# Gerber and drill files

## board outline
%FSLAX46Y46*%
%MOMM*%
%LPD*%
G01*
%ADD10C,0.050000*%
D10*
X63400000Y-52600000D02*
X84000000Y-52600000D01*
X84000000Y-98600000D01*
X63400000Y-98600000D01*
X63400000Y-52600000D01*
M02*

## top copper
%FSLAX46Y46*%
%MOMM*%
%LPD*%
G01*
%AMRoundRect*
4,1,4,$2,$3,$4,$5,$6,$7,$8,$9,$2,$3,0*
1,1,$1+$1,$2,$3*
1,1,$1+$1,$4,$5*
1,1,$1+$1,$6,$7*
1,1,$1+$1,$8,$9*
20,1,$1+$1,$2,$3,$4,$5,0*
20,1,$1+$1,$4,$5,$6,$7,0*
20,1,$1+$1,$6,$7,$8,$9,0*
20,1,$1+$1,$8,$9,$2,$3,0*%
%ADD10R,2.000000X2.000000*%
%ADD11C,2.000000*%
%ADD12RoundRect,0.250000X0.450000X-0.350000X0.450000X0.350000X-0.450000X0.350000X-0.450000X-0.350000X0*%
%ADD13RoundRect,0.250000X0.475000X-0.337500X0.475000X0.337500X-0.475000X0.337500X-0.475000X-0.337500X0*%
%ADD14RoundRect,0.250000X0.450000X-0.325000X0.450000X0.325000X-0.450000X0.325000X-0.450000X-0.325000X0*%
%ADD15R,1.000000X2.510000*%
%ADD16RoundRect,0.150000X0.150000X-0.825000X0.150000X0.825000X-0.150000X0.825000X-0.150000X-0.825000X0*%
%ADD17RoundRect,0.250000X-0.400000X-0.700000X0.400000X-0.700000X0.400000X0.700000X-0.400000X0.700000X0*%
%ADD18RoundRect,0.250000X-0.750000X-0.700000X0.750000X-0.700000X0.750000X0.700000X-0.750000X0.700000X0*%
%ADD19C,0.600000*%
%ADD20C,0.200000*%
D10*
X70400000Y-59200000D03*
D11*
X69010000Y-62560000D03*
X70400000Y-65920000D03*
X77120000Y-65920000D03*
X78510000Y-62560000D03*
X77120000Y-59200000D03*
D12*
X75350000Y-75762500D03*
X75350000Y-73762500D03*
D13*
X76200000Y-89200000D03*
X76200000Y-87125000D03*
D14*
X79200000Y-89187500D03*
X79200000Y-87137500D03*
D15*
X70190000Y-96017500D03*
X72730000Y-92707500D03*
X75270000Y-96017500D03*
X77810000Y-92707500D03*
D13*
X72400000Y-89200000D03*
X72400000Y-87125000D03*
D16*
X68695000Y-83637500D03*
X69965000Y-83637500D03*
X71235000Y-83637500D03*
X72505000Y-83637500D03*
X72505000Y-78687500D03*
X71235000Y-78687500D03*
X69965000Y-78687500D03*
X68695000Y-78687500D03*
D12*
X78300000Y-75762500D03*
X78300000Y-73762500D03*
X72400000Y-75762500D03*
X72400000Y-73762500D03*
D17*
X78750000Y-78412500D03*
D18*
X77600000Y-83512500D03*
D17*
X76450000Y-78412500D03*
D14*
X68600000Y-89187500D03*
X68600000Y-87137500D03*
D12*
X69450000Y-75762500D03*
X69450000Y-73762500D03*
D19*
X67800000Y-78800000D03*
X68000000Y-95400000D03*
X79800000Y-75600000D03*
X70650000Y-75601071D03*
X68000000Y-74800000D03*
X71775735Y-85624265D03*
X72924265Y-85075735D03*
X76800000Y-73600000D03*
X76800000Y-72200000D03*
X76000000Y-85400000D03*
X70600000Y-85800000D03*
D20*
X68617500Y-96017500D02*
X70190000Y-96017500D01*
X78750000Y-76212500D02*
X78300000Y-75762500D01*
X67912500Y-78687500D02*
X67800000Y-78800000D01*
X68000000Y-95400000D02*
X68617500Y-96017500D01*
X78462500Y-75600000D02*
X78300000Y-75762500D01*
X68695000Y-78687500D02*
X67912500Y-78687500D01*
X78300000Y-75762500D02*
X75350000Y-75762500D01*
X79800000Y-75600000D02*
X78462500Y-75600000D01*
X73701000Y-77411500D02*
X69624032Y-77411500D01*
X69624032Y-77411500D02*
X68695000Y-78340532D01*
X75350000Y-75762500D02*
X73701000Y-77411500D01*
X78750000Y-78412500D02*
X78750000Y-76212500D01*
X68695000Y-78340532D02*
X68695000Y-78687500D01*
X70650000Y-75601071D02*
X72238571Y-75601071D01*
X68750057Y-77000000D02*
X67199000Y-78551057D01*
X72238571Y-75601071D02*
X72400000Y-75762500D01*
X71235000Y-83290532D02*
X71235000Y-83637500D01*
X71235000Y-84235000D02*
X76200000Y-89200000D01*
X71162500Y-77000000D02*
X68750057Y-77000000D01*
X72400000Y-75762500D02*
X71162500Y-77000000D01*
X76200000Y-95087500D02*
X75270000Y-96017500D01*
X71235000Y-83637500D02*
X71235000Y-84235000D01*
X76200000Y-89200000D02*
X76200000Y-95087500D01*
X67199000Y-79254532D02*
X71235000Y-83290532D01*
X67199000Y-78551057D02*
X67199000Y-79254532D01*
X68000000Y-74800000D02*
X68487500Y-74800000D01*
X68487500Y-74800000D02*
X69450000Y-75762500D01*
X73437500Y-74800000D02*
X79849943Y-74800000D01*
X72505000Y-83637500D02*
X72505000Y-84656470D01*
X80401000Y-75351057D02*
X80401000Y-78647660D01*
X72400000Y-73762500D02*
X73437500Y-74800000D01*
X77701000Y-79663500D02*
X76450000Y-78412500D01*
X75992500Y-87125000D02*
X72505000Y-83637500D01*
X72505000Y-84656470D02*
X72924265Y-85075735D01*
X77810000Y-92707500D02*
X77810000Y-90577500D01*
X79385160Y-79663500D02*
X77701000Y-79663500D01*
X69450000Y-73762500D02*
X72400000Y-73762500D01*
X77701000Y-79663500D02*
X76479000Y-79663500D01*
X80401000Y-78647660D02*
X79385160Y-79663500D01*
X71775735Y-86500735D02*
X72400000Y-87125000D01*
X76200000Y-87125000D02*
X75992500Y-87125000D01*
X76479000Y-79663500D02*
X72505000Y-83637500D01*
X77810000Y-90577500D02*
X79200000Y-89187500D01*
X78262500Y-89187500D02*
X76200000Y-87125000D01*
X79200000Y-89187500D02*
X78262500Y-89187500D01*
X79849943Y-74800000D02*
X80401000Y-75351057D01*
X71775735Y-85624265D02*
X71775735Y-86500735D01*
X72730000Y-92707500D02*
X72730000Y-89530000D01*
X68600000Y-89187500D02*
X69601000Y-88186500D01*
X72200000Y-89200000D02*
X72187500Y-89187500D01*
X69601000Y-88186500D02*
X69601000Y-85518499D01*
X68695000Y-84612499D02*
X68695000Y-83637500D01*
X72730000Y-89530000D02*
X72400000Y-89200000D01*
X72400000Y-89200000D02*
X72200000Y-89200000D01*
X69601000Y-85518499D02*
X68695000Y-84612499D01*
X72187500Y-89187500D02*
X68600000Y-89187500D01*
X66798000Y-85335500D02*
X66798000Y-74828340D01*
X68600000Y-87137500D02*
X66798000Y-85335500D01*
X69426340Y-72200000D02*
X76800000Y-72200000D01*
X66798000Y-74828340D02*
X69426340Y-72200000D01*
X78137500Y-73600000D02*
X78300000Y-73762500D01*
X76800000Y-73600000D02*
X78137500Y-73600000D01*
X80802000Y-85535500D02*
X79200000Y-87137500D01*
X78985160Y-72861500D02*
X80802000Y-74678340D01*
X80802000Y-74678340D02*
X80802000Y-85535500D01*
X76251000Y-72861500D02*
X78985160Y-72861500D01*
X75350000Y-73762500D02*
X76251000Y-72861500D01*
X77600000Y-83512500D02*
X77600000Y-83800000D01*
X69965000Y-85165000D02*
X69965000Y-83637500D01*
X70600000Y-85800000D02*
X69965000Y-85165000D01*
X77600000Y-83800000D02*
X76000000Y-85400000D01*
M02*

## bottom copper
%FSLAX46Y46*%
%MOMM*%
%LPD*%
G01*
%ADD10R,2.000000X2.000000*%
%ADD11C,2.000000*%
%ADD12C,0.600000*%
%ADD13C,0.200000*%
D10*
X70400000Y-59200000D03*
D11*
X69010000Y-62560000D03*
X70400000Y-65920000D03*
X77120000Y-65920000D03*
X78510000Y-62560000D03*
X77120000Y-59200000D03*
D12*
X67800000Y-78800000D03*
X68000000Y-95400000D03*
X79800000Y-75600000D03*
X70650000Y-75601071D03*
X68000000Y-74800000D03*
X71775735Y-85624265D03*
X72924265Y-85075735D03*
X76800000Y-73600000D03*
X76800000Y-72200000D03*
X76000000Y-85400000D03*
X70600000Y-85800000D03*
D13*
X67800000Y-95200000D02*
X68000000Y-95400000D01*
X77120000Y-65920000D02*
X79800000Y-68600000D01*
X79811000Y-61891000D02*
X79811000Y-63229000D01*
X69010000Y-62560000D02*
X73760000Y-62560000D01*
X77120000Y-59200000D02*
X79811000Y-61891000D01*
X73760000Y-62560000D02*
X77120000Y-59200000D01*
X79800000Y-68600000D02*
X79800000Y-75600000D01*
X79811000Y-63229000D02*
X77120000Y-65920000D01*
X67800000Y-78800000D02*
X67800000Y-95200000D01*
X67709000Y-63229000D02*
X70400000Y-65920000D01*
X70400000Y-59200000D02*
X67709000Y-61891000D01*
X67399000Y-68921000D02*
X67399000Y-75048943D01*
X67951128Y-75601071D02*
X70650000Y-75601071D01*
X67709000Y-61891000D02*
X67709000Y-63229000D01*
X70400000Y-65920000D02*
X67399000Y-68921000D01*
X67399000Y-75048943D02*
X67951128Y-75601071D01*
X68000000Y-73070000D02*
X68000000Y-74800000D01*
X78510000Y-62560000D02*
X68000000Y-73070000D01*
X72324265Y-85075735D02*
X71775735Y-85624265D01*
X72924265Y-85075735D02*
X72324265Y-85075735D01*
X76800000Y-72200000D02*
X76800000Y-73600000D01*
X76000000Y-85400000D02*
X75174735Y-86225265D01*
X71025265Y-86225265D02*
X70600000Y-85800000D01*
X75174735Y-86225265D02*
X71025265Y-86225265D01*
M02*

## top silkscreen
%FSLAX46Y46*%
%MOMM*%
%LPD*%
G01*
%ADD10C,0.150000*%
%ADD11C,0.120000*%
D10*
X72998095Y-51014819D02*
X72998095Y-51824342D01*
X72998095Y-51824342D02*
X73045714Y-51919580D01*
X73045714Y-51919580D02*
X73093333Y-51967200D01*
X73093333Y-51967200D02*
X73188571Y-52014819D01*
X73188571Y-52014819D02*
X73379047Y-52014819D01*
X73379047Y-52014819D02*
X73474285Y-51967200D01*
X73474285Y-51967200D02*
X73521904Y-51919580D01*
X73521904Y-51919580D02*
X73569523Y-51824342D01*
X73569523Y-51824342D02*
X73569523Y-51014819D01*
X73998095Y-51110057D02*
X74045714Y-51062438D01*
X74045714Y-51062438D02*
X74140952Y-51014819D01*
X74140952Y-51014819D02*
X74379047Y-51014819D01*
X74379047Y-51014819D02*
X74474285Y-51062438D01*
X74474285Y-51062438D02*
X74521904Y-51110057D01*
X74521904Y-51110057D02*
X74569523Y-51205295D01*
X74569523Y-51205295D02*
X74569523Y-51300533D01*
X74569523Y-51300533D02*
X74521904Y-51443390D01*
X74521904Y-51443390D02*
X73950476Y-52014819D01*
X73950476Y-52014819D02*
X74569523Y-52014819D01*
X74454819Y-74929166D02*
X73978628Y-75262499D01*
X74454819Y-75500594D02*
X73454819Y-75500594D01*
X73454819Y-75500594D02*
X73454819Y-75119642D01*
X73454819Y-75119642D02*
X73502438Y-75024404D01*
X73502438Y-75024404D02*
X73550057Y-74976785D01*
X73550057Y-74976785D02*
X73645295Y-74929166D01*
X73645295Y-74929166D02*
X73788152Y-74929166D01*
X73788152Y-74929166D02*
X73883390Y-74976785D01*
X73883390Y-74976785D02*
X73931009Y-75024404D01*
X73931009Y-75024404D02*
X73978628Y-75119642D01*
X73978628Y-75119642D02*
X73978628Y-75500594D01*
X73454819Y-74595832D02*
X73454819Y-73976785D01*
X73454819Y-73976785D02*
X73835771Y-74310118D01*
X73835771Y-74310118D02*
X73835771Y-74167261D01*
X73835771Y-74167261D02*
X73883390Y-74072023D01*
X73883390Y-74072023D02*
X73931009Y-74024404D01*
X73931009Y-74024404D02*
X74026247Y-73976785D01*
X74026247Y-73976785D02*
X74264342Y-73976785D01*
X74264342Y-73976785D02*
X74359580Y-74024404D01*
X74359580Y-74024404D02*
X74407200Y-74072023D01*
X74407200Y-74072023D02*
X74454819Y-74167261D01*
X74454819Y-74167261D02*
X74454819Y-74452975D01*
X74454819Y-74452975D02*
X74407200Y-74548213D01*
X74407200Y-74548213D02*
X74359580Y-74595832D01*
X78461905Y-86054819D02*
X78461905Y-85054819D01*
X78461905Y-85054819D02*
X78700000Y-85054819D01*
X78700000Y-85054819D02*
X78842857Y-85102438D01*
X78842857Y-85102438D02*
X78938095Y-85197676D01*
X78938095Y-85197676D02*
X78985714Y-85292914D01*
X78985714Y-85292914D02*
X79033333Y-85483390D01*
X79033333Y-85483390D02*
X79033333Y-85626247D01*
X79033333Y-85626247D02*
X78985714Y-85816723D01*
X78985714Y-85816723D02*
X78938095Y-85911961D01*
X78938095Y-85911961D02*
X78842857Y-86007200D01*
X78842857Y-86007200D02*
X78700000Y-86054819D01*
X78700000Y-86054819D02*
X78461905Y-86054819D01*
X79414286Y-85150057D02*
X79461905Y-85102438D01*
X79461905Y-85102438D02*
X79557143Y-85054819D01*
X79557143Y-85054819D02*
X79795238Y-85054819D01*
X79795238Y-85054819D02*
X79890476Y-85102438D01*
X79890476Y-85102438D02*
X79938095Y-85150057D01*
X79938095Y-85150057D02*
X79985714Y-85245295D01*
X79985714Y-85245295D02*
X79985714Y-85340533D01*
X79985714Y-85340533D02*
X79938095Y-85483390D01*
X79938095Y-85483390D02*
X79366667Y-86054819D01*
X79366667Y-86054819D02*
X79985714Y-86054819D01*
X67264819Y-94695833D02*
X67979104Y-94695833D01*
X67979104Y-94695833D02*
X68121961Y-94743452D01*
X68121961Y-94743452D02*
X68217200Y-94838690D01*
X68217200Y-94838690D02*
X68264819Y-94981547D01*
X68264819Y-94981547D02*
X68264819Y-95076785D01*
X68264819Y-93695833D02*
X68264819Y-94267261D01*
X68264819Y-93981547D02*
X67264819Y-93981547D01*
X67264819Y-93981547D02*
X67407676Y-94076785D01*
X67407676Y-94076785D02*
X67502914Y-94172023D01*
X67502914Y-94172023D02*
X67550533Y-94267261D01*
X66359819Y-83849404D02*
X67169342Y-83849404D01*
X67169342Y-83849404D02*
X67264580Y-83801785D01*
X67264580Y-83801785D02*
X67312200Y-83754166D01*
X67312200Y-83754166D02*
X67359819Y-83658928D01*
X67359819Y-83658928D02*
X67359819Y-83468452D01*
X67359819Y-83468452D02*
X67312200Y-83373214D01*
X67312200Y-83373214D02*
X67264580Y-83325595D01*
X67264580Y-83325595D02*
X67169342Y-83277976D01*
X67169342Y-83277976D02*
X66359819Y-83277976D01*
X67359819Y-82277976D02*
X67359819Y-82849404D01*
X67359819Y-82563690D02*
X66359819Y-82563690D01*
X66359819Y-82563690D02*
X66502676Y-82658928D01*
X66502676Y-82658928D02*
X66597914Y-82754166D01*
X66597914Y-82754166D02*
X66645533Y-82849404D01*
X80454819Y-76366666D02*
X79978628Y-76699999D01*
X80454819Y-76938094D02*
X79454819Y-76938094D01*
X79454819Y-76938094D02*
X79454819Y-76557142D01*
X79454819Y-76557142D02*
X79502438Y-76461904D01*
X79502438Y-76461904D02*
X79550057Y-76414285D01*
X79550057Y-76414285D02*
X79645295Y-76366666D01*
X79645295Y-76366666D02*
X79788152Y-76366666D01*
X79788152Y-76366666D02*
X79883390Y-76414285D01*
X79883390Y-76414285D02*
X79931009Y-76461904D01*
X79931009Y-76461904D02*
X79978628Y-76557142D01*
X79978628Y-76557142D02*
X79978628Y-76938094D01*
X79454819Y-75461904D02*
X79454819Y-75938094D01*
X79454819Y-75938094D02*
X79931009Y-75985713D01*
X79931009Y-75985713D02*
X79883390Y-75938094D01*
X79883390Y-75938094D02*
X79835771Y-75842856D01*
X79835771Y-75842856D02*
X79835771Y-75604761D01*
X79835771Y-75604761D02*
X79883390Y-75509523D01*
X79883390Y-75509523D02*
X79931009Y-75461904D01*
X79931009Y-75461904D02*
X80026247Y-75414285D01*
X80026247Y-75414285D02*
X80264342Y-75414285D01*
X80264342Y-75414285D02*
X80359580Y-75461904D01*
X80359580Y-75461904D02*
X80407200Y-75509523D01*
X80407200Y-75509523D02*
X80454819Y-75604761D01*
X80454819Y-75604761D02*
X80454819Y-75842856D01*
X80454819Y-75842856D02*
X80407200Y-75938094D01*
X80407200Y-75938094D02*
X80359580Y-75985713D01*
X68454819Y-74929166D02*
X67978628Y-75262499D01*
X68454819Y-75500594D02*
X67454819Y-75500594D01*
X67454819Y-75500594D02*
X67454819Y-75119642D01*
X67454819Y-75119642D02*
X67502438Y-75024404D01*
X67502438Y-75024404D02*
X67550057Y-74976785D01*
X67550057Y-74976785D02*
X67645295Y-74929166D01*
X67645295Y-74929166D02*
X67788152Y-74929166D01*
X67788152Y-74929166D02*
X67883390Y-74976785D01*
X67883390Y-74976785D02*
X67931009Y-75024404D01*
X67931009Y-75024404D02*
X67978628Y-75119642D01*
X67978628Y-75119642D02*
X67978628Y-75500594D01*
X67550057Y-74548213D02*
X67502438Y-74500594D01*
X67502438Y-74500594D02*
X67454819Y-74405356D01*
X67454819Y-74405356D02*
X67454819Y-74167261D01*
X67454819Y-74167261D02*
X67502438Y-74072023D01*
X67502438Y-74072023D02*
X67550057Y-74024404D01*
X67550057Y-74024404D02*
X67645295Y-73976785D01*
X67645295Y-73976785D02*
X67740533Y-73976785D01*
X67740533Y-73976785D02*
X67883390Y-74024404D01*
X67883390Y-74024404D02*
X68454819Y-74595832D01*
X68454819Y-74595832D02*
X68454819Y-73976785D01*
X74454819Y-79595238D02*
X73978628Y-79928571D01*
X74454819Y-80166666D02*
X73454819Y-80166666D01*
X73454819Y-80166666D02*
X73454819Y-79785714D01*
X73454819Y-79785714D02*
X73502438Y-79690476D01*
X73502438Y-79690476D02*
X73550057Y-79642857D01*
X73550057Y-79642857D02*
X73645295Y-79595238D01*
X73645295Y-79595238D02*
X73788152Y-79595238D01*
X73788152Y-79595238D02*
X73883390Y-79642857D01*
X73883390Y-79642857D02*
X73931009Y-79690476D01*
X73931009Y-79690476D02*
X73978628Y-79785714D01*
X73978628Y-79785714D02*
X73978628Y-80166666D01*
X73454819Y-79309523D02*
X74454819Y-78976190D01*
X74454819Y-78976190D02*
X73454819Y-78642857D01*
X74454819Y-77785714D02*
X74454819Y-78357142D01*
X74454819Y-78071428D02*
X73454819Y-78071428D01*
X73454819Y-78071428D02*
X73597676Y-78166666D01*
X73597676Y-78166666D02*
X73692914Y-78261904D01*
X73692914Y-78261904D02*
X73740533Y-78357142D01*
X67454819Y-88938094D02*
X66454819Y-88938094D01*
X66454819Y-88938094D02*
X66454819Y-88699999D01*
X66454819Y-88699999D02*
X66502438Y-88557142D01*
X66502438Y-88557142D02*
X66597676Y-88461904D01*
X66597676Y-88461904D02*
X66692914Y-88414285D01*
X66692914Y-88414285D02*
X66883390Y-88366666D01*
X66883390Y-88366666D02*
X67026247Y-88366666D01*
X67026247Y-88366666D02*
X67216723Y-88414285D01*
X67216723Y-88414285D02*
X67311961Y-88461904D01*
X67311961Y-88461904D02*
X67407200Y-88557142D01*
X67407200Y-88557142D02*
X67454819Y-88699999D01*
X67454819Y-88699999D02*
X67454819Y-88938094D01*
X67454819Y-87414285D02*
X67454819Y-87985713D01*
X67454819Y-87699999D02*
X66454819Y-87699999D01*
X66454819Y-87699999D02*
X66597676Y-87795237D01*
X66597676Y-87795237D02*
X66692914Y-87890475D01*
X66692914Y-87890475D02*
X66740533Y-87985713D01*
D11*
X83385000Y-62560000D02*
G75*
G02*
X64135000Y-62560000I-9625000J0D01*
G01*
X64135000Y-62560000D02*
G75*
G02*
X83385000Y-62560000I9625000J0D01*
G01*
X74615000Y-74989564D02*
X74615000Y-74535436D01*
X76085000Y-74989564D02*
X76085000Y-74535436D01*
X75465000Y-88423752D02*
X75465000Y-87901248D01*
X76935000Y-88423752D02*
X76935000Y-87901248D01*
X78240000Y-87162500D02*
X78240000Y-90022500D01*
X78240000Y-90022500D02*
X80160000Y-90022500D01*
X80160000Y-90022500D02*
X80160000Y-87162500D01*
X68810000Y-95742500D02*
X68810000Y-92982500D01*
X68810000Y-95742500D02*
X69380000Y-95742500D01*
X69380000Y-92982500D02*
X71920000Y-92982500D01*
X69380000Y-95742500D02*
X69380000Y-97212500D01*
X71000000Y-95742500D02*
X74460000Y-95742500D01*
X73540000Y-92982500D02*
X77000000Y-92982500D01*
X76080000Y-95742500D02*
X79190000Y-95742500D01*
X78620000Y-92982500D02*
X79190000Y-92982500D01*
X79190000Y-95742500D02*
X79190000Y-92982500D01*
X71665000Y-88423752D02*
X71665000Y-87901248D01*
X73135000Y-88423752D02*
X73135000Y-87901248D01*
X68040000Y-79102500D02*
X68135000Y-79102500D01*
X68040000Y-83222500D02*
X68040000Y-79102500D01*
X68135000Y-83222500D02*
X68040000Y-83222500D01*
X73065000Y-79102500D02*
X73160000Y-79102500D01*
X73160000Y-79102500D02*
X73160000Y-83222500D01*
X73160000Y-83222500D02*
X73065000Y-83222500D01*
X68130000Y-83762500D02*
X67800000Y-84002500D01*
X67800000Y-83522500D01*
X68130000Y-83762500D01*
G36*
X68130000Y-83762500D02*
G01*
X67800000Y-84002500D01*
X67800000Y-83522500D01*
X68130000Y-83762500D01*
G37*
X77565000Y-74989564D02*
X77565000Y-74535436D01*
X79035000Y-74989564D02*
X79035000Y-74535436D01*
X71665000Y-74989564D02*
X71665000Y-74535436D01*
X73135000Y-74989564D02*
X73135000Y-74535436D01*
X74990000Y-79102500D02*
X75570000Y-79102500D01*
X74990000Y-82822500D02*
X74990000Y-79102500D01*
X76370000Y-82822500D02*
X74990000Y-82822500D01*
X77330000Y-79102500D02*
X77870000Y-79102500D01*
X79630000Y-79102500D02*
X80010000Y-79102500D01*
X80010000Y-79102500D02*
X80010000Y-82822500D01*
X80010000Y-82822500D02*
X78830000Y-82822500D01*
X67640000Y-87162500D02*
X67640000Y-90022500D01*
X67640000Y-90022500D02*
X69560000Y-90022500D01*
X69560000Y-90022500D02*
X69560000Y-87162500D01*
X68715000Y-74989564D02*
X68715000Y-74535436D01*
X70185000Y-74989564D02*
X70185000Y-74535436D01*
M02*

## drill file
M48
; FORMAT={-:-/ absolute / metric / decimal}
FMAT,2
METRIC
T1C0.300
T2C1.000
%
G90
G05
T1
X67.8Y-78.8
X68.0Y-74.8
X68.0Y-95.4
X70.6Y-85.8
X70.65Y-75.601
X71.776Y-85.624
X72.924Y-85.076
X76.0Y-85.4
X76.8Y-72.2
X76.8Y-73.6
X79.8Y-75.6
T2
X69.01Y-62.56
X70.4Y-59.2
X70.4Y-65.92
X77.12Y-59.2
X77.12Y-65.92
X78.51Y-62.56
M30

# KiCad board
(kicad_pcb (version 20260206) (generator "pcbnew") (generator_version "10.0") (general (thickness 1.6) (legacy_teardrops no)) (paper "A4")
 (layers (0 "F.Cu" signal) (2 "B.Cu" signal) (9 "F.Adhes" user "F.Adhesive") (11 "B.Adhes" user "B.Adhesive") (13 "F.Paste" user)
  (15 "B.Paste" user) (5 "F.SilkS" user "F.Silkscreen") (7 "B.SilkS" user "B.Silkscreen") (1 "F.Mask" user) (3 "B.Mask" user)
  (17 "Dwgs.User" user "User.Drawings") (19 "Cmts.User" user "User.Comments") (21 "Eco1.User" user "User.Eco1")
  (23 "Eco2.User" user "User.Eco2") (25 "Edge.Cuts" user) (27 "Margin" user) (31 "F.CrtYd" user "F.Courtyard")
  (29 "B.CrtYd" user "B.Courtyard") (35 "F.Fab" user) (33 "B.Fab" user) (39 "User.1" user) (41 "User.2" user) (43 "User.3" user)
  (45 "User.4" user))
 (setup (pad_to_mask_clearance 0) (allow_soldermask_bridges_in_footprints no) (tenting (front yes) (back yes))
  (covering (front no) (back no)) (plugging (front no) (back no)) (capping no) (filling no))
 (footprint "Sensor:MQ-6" (layer "F.Cu") (at 70.4 59.2)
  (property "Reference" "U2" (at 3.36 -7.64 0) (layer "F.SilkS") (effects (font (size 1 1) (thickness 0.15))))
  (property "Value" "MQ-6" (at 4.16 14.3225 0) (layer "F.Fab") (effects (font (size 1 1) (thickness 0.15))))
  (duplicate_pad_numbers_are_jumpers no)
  (fp_circle (center 3.36 3.36) (end 12.985 3.36) (stroke (width 0.12) (type solid)) (fill no) (layer "F.SilkS"))
  (pad "1" thru_hole rect (at 0 0) (size 2 2) (drill 1) (layers "*.Cu" "*.Mask") (remove_unused_layers no) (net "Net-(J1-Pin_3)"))
  (pad "2" thru_hole circle (at -1.39 3.36) (size 2 2) (drill 1) (layers "*.Cu" "*.Mask") (remove_unused_layers no) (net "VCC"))
  (pad "3" thru_hole circle (at 0 6.72 90) (size 2 2) (drill 1) (layers "*.Cu" "*.Mask") (remove_unused_layers no) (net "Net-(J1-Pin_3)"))
  (pad "4" thru_hole circle (at 6.72 6.72 180) (size 2 2) (drill 1) (layers "*.Cu" "*.Mask") (remove_unused_layers no) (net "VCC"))
  (pad "5" thru_hole circle (at 8.11 3.36) (size 2 2) (drill 1) (layers "*.Cu" "*.Mask") (remove_unused_layers no) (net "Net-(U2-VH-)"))
  (pad "6" thru_hole circle (at 6.72 0 270) (size 2 2) (drill 1) (layers "*.Cu" "*.Mask") (remove_unused_layers no) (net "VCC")))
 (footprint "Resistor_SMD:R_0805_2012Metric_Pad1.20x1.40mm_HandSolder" (layer "F.Cu") (at 75.35 74.7625 90)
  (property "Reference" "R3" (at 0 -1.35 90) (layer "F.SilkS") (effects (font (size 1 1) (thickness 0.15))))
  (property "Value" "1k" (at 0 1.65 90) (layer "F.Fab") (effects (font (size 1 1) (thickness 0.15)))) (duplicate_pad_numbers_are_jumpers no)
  (fp_line (start -0.227064 -0.735) (end 0.227064 -0.735) (stroke (width 0.12) (type solid)) (layer "F.SilkS"))
  (fp_line (start -0.227064 0.735) (end 0.227064 0.735) (stroke (width 0.12) (type solid)) (layer "F.SilkS"))
  (pad "1" smd roundrect (at -1 0 90) (size 1.2 1.4) (layers "F.Cu" "F.Mask" "F.Paste") (roundrect_rratio 0.208333) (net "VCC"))
  (pad "2" smd roundrect (at 1 0 90) (size 1.2 1.4) (layers "F.Cu" "F.Mask" "F.Paste") (roundrect_rratio 0.208333) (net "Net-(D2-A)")))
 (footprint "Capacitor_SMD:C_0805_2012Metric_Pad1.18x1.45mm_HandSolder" (layer "F.Cu") (at 76.2 88.1625 90)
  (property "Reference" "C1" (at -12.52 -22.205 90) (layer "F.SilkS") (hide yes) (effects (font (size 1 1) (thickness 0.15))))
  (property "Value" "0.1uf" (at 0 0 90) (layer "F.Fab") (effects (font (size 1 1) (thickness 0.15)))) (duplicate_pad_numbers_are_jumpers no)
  (fp_line (start -0.261252 -0.735) (end 0.261252 -0.735) (stroke (width 0.12) (type solid)) (layer "F.SilkS"))
  (fp_line (start -0.261252 0.735) (end 0.261252 0.735) (stroke (width 0.12) (type solid)) (layer "F.SilkS"))
  (pad "1" smd roundrect (at -1.0375 0 90) (size 1.175 1.45) (layers "F.Cu" "F.Mask" "F.Paste") (roundrect_rratio 0.212766)
   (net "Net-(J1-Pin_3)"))
  (pad "2" smd roundrect (at 1.0375 0 90) (size 1.175 1.45) (layers "F.Cu" "F.Mask" "F.Paste") (roundrect_rratio 0.212766) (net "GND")))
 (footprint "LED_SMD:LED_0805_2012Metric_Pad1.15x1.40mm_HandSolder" (layer "F.Cu") (at 79.2 88.1625 90)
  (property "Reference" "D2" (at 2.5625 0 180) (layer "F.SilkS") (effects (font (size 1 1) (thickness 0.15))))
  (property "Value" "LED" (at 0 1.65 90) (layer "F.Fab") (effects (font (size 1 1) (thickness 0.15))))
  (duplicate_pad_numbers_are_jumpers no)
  (fp_line (start 1 -0.96) (end -1.86 -0.96) (stroke (width 0.12) (type solid)) (layer "F.SilkS"))
  (fp_line (start -1.86 -0.96) (end -1.86 0.96) (stroke (width 0.12) (type solid)) (layer "F.SilkS"))
  (fp_line (start -1.86 0.96) (end 1 0.96) (stroke (width 0.12) (type solid)) (layer "F.SilkS"))
  (pad "1" smd roundrect (at -1.025 0 90) (size 1.15 1.4) (layers "F.Cu" "F.Mask" "F.Paste") (roundrect_rratio 0.217391) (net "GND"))
  (pad "2" smd roundrect (at 1.025 0 90) (size 1.15 1.4) (layers "F.Cu" "F.Mask" "F.Paste") (roundrect_rratio 0.217391) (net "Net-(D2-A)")))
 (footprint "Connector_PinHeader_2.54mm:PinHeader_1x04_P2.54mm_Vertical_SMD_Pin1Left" (layer "F.Cu") (at 74 94.3625 90)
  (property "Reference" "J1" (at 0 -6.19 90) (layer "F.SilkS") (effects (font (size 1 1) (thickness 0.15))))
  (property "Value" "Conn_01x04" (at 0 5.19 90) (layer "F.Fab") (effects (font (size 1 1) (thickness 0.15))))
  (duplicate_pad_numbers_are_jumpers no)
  (fp_line (start -1.38 -5.19) (end 1.38 -5.19) (stroke (width 0.12) (type solid)) (layer "F.SilkS"))
  (fp_line (start -1.38 -5.19) (end -1.38 -4.62) (stroke (width 0.12) (type solid)) (layer "F.SilkS"))
  (fp_line (start 1.38 -4.62) (end 1.38 -2.08) (stroke (width 0.12) (type solid)) (layer "F.SilkS"))
  (fp_line (start -1.38 -4.62) (end -2.85 -4.62) (stroke (width 0.12) (type solid)) (layer "F.SilkS"))
  (fp_line (start -1.38 -3) (end -1.38 0.46) (stroke (width 0.12) (type solid)) (layer "F.SilkS"))
  (fp_line (start 1.38 -0.46) (end 1.38 3) (stroke (width 0.12) (type solid)) (layer "F.SilkS"))
  (fp_line (start -1.38 2.08) (end -1.38 5.19) (stroke (width 0.12) (type solid)) (layer "F.SilkS"))
  (fp_line (start 1.38 4.62) (end 1.38 5.19) (stroke (width 0.12) (type solid)) (layer "F.SilkS"))
  (fp_line (start -1.38 5.19) (end 1.38 5.19) (stroke (width 0.12) (type solid)) (layer "F.SilkS"))
  (pad "1" smd rect (at -1.655 -3.81 90) (size 2.51 1) (layers "F.Cu" "F.Mask" "F.Paste") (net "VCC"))
  (pad "2" smd rect (at 1.655 -1.27 90) (size 2.51 1) (layers "F.Cu" "F.Mask" "F.Paste") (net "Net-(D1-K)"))
  (pad "3" smd rect (at -1.655 1.27 90) (size 2.51 1) (layers "F.Cu" "F.Mask" "F.Paste") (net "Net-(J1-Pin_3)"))
  (pad "4" smd rect (at 1.655 3.81 90) (size 2.51 1) (layers "F.Cu" "F.Mask" "F.Paste") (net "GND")))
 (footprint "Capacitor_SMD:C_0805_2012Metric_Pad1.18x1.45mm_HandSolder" (layer "F.Cu") (at 72.4 88.1625 90)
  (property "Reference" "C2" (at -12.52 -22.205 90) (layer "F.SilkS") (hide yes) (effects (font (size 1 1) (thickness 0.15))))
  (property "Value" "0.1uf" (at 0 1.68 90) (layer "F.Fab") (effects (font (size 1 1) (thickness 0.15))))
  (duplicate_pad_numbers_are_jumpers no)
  (fp_line (start -0.261252 -0.735) (end 0.261252 -0.735) (stroke (width 0.12) (type solid)) (layer "F.SilkS"))
  (fp_line (start -0.261252 0.735) (end 0.261252 0.735) (stroke (width 0.12) (type solid)) (layer "F.SilkS"))
  (pad "1" smd roundrect (at -1.0375 0 90) (size 1.175 1.45) (layers "F.Cu" "F.Mask" "F.Paste") (roundrect_rratio 0.212766)
   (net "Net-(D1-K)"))
  (pad "2" smd roundrect (at 1.0375 0 90) (size 1.175 1.45) (layers "F.Cu" "F.Mask" "F.Paste") (roundrect_rratio 0.212766) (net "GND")))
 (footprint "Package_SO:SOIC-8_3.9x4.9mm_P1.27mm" (layer "F.Cu") (at 70.6 81.1625 90)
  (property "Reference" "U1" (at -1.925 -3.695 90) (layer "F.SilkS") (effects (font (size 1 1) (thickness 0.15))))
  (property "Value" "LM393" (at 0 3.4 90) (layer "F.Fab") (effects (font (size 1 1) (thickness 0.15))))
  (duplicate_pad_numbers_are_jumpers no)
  (fp_line (start 2.06 -2.56) (end 2.06 -2.465) (stroke (width 0.12) (type solid)) (layer "F.SilkS"))
  (fp_line (start -2.06 -2.56) (end 2.06 -2.56) (stroke (width 0.12) (type solid)) (layer "F.SilkS"))
  (fp_line (start -2.06 -2.465) (end -2.06 -2.56) (stroke (width 0.12) (type solid)) (layer "F.SilkS"))
  (fp_line (start 2.06 2.465) (end 2.06 2.56) (stroke (width 0.12) (type solid)) (layer "F.SilkS"))
  (fp_line (start 2.06 2.56) (end -2.06 2.56) (stroke (width 0.12) (type solid)) (layer "F.SilkS"))
  (fp_line (start -2.06 2.56) (end -2.06 2.465) (stroke (width 0.12) (type solid)) (layer "F.SilkS"))
  (fp_poly (pts (xy -2.6 -2.47) (xy -2.84 -2.8) (xy -2.36 -2.8)) (stroke (width 0.12) (type solid)) (fill yes) (layer "F.SilkS"))
  (pad "1" smd roundrect (at -2.475 -1.905 90) (size 1.95 0.6) (layers "F.Cu" "F.Mask" "F.Paste") (roundrect_rratio 0.25) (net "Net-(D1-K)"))
  (pad "2" smd roundrect (at -2.475 -0.635 90) (size 1.95 0.6) (layers "F.Cu" "F.Mask" "F.Paste") (roundrect_rratio 0.25)
   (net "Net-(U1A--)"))
  (pad "3" smd roundrect (at -2.475 0.635 90) (size 1.95 0.6) (layers "F.Cu" "F.Mask" "F.Paste") (roundrect_rratio 0.25)
   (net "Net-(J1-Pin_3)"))
  (pad "4" smd roundrect (at -2.475 1.905 90) (size 1.95 0.6) (layers "F.Cu" "F.Mask" "F.Paste") (roundrect_rratio 0.25) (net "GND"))
  (pad "5" smd roundrect (at 2.475 1.905 90) (size 1.95 0.6) (layers "F.Cu" "F.Mask" "F.Paste") (roundrect_rratio 0.25))
  (pad "6" smd roundrect (at 2.475 0.635 90) (size 1.95 0.6) (layers "F.Cu" "F.Mask" "F.Paste") (roundrect_rratio 0.25))
  (pad "7" smd roundrect (at 2.475 -0.635 90) (size 1.95 0.6) (layers "F.Cu" "F.Mask" "F.Paste") (roundrect_rratio 0.25))
  (pad "8" smd roundrect (at 2.475 -1.905 90) (size 1.95 0.6) (layers "F.Cu" "F.Mask" "F.Paste") (roundrect_rratio 0.25) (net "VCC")))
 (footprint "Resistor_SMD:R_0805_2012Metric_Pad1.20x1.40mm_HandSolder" (layer "F.Cu") (at 78.3 74.7625 90)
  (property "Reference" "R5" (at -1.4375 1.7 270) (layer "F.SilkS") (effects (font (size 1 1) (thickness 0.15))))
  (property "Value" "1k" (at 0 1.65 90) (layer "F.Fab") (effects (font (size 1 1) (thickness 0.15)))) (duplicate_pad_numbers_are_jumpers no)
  (fp_line (start -0.227064 -0.735) (end 0.227064 -0.735) (stroke (width 0.12) (type solid)) (layer "F.SilkS"))
  (fp_line (start -0.227064 0.735) (end 0.227064 0.735) (stroke (width 0.12) (type solid)) (layer "F.SilkS"))
  (pad "1" smd roundrect (at -1 0 90) (size 1.2 1.4) (layers "F.Cu" "F.Mask" "F.Paste") (roundrect_rratio 0.208333) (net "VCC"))
  (pad "2" smd roundrect (at 1 0 90) (size 1.2 1.4) (layers "F.Cu" "F.Mask" "F.Paste") (roundrect_rratio 0.208333) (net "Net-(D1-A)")))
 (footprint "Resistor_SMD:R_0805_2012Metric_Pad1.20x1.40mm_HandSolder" (layer "F.Cu") (at 72.4 74.7625 90)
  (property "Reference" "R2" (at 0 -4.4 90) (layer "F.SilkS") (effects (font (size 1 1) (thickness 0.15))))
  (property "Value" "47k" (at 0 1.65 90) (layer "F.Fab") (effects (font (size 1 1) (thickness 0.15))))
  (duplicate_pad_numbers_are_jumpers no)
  (fp_line (start -0.227064 -0.735) (end 0.227064 -0.735) (stroke (width 0.12) (type solid)) (layer "F.SilkS"))
  (fp_line (start -0.227064 0.735) (end 0.227064 0.735) (stroke (width 0.12) (type solid)) (layer "F.SilkS"))
  (pad "1" smd roundrect (at -1 0 90) (size 1.2 1.4) (layers "F.Cu" "F.Mask" "F.Paste") (roundrect_rratio 0.208333) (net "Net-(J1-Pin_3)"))
  (pad "2" smd roundrect (at 1 0 90) (size 1.2 1.4) (layers "F.Cu" "F.Mask" "F.Paste") (roundrect_rratio 0.208333) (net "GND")))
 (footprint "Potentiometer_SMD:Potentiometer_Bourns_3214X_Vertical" (layer "F.Cu") (at 77.6 80.9625)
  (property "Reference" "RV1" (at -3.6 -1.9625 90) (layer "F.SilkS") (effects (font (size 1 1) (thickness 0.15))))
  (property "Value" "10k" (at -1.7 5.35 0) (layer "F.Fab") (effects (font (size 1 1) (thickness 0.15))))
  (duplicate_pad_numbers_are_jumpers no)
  (fp_line (start -2.61 -1.86) (end -2.03 -1.86) (stroke (width 0.12) (type solid)) (layer "F.SilkS"))
  (fp_line (start -2.61 1.86) (end -2.61 -1.86) (stroke (width 0.12) (type solid)) (layer "F.SilkS"))
  (fp_line (start -1.23 1.86) (end -2.61 1.86) (stroke (width 0.12) (type solid)) (layer "F.SilkS"))
  (fp_line (start -0.27 -1.86) (end 0.27 -1.86) (stroke (width 0.12) (type solid)) (layer "F.SilkS"))
  (fp_line (start 2.03 -1.86) (end 2.41 -1.86) (stroke (width 0.12) (type solid)) (layer "F.SilkS"))
  (fp_line (start 2.41 -1.86) (end 2.41 1.86) (stroke (width 0.12) (type solid)) (layer "F.SilkS"))
  (fp_line (start 2.41 1.86) (end 1.23 1.86) (stroke (width 0.12) (type solid)) (layer "F.SilkS"))
  (pad "1" smd roundrect (at 1.15 -2.55) (size 1.3 1.9) (layers "F.Cu" "F.Mask" "F.Paste") (roundrect_rratio 0.192308) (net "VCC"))
  (pad "2" smd roundrect (at 0 2.55) (size 2 1.9) (layers "F.Cu" "F.Mask" "F.Paste") (roundrect_rratio 0.131579) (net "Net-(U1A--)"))
  (pad "3" smd roundrect (at -1.15 -2.55) (size 1.3 1.9) (layers "F.Cu" "F.Mask" "F.Paste") (roundrect_rratio 0.192308) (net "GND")))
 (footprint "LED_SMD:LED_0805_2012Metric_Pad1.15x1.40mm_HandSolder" (layer "F.Cu") (at 68.6 88.1625 90)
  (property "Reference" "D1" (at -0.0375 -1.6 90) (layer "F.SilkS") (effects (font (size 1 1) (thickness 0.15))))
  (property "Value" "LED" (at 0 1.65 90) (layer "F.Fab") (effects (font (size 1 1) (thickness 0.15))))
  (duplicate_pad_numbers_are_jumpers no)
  (fp_line (start 1 -0.96) (end -1.86 -0.96) (stroke (width 0.12) (type solid)) (layer "F.SilkS"))
  (fp_line (start -1.86 -0.96) (end -1.86 0.96) (stroke (width 0.12) (type solid)) (layer "F.SilkS"))
  (fp_line (start -1.86 0.96) (end 1 0.96) (stroke (width 0.12) (type solid)) (layer "F.SilkS"))
  (pad "1" smd roundrect (at -1.025 0 90) (size 1.15 1.4) (layers "F.Cu" "F.Mask" "F.Paste") (roundrect_rratio 0.217391) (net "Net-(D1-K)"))
  (pad "2" smd roundrect (at 1.025 0 90) (size 1.15 1.4) (layers "F.Cu" "F.Mask" "F.Paste") (roundrect_rratio 0.217391) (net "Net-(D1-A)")))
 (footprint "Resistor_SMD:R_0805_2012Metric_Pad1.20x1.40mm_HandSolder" (layer "F.Cu") (at 69.45 74.7625 90)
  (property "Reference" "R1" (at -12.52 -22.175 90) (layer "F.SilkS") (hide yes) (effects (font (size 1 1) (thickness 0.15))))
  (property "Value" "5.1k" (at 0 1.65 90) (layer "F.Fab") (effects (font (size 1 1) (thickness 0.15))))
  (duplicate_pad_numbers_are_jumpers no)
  (fp_line (start -0.227064 -0.735) (end 0.227064 -0.735) (stroke (width 0.12) (type solid)) (layer "F.SilkS"))
  (fp_line (start -0.227064 0.735) (end 0.227064 0.735) (stroke (width 0.12) (type solid)) (layer "F.SilkS"))
  (pad "1" smd roundrect (at -1 0 90) (size 1.2 1.4) (layers "F.Cu" "F.Mask" "F.Paste") (roundrect_rratio 0.208333) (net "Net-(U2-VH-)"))
  (pad "2" smd roundrect (at 1 0 90) (size 1.2 1.4) (layers "F.Cu" "F.Mask" "F.Paste") (roundrect_rratio 0.208333) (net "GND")))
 (gr_rect (start 63.4 52.6) (end 84 98.6) (stroke (width 0.05) (type default)) (fill no) (layer "Edge.Cuts"))
 (segment (start 68.6175 96.0175) (end 70.19 96.0175) (width 0.2) (layer "F.Cu") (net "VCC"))
 (segment (start 78.75 76.2125) (end 78.3 75.7625) (width 0.2) (layer "F.Cu") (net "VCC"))
 (segment (start 67.9125 78.6875) (end 67.8 78.8) (width 0.2) (layer "F.Cu") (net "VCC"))
 (segment (start 68 95.4) (end 68.6175 96.0175) (width 0.2) (layer "F.Cu") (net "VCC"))
 (segment (start 78.4625 75.6) (end 78.3 75.7625) (width 0.2) (layer "F.Cu") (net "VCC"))
 (segment (start 68.695 78.6875) (end 67.9125 78.6875) (width 0.2) (layer "F.Cu") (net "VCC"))
 (segment (start 78.3 75.7625) (end 75.35 75.7625) (width 0.2) (layer "F.Cu") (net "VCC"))
 (segment (start 79.8 75.6) (end 78.4625 75.6) (width 0.2) (layer "F.Cu") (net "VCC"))
 (segment (start 73.701 77.4115) (end 69.624032 77.4115) (width 0.2) (layer "F.Cu") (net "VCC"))
 (segment (start 69.624032 77.4115) (end 68.695 78.340532) (width 0.2) (layer "F.Cu") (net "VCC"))
 (segment (start 75.35 75.7625) (end 73.701 77.4115) (width 0.2) (layer "F.Cu") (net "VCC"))
 (segment (start 78.75 78.4125) (end 78.75 76.2125) (width 0.2) (layer "F.Cu") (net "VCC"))
 (segment (start 68.695 78.340532) (end 68.695 78.6875) (width 0.2) (layer "F.Cu") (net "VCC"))
 (via (at 67.8 78.8) (size 0.6) (drill 0.3) (layers "F.Cu" "B.Cu") (capping no) (covering (front no) (back no))
  (plugging (front no) (back no)) (filling no) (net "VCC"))
 (via (at 68 95.4) (size 0.6) (drill 0.3) (layers "F.Cu" "B.Cu") (capping no) (covering (front no) (back no))
  (plugging (front no) (back no)) (filling no) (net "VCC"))
 (via (at 79.8 75.6) (size 0.6) (drill 0.3) (layers "F.Cu" "B.Cu") (capping no) (covering (front no) (back no))
  (plugging (front no) (back no)) (filling no) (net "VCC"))
 (segment (start 67.8 95.2) (end 68 95.4) (width 0.2) (layer "B.Cu") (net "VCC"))
 (segment (start 77.12 65.92) (end 79.8 68.6) (width 0.2) (layer "B.Cu") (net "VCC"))
 (segment (start 79.811 61.891) (end 79.811 63.229) (width 0.2) (layer "B.Cu") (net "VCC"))
 (segment (start 69.01 62.56) (end 73.76 62.56) (width 0.2) (layer "B.Cu") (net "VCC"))
 (segment (start 77.12 59.2) (end 79.811 61.891) (width 0.2) (layer "B.Cu") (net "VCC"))
 (segment (start 73.76 62.56) (end 77.12 59.2) (width 0.2) (layer "B.Cu") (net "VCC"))
 (segment (start 79.8 68.6) (end 79.8 75.6) (width 0.2) (layer "B.Cu") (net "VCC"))
 (segment (start 79.811 63.229) (end 77.12 65.92) (width 0.2) (layer "B.Cu") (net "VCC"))
 (segment (start 67.8 78.8) (end 67.8 95.2) (width 0.2) (layer "B.Cu") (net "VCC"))
 (segment (start 70.65 75.601071) (end 72.238571 75.601071) (width 0.2) (layer "F.Cu") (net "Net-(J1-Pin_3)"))
 (segment (start 68.750057 77) (end 67.199 78.551057) (width 0.2) (layer "F.Cu") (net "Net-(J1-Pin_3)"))
 (segment (start 72.238571 75.601071) (end 72.4 75.7625) (width 0.2) (layer "F.Cu") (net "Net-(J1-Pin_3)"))
 (segment (start 71.235 83.290532) (end 71.235 83.6375) (width 0.2) (layer "F.Cu") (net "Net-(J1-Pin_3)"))
 (segment (start 71.235 84.235) (end 76.2 89.2) (width 0.2) (layer "F.Cu") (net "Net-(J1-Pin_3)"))
 (segment (start 71.1625 77) (end 68.750057 77) (width 0.2) (layer "F.Cu") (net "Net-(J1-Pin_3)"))
 (segment (start 72.4 75.7625) (end 71.1625 77) (width 0.2) (layer "F.Cu") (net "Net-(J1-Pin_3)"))
 (segment (start 76.2 95.0875) (end 75.27 96.0175) (width 0.2) (layer "F.Cu") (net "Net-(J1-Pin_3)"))
 (segment (start 71.235 83.6375) (end 71.235 84.235) (width 0.2) (layer "F.Cu") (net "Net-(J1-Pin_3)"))
 (segment (start 76.2 89.2) (end 76.2 95.0875) (width 0.2) (layer "F.Cu") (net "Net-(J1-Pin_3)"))
 (segment (start 67.199 79.254532) (end 71.235 83.290532) (width 0.2) (layer "F.Cu") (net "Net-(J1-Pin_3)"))
 (segment (start 67.199 78.551057) (end 67.199 79.254532) (width 0.2) (layer "F.Cu") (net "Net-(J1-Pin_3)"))
 (via (at 70.65 75.601071) (size 0.6) (drill 0.3) (layers "F.Cu" "B.Cu") (capping no) (covering (front no) (back no))
  (plugging (front no) (back no)) (filling no) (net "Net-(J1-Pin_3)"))
 (segment (start 67.709 63.229) (end 70.4 65.92) (width 0.2) (layer "B.Cu") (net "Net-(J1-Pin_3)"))
 (segment (start 70.4 59.2) (end 67.709 61.891) (width 0.2) (layer "B.Cu") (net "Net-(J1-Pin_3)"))
 (segment (start 67.399 68.921) (end 67.399 75.048943) (width 0.2) (layer "B.Cu") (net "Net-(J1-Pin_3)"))
 (segment (start 67.951128 75.601071) (end 70.65 75.601071) (width 0.2) (layer "B.Cu") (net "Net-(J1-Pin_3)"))
 (segment (start 67.709 61.891) (end 67.709 63.229) (width 0.2) (layer "B.Cu") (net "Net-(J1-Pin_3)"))
 (segment (start 70.4 65.92) (end 67.399 68.921) (width 0.2) (layer "B.Cu") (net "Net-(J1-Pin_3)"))
 (segment (start 67.399 75.048943) (end 67.951128 75.601071) (width 0.2) (layer "B.Cu") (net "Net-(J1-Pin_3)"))
 (segment (start 68 74.8) (end 68.4875 74.8) (width 0.2) (layer "F.Cu") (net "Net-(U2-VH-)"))
 (segment (start 68.4875 74.8) (end 69.45 75.7625) (width 0.2) (layer "F.Cu") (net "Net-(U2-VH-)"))
 (via (at 68 74.8) (size 0.6) (drill 0.3) (layers "F.Cu" "B.Cu") (capping no) (covering (front no) (back no))
  (plugging (front no) (back no)) (filling no) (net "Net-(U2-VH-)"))
 (segment (start 68 73.07) (end 68 74.8) (width 0.2) (layer "B.Cu") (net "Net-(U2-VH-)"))
 (segment (start 78.51 62.56) (end 68 73.07) (width 0.2) (layer "B.Cu") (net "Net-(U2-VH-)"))
 (segment (start 73.4375 74.8) (end 79.849943 74.8) (width 0.2) (layer "F.Cu") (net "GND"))
 (segment (start 72.505 83.6375) (end 72.505 84.65647) (width 0.2) (layer "F.Cu") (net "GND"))
 (segment (start 80.401 75.351057) (end 80.401 78.64766) (width 0.2) (layer "F.Cu") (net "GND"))
 (segment (start 72.4 73.7625) (end 73.4375 74.8) (width 0.2) (layer "F.Cu") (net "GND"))
 (segment (start 77.701 79.6635) (end 76.45 78.4125) (width 0.2) (layer "F.Cu") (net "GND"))
 (segment (start 75.9925 87.125) (end 72.505 83.6375) (width 0.2) (layer "F.Cu") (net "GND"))
 (segment (start 72.505 84.65647) (end 72.924265 85.075735) (width 0.2) (layer "F.Cu") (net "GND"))
 (segment (start 77.81 92.7075) (end 77.81 90.5775) (width 0.2) (layer "F.Cu") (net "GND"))
 (segment (start 79.38516 79.6635) (end 77.701 79.6635) (width 0.2) (layer "F.Cu") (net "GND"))
 (segment (start 69.45 73.7625) (end 72.4 73.7625) (width 0.2) (layer "F.Cu") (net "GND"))
 (segment (start 77.701 79.6635) (end 76.479 79.6635) (width 0.2) (layer "F.Cu") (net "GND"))
 (segment (start 80.401 78.64766) (end 79.38516 79.6635) (width 0.2) (layer "F.Cu") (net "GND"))
 (segment (start 71.775735 86.500735) (end 72.4 87.125) (width 0.2) (layer "F.Cu") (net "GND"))
 (segment (start 76.2 87.125) (end 75.9925 87.125) (width 0.2) (layer "F.Cu") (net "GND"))
 (segment (start 76.479 79.6635) (end 72.505 83.6375) (width 0.2) (layer "F.Cu") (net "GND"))
 (segment (start 77.81 90.5775) (end 79.2 89.1875) (width 0.2) (layer "F.Cu") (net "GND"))
 (segment (start 78.2625 89.1875) (end 76.2 87.125) (width 0.2) (layer "F.Cu") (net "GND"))
 (segment (start 79.2 89.1875) (end 78.2625 89.1875) (width 0.2) (layer "F.Cu") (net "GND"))
 (segment (start 79.849943 74.8) (end 80.401 75.351057) (width 0.2) (layer "F.Cu") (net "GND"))
 (segment (start 71.775735 85.624265) (end 71.775735 86.500735) (width 0.2) (layer "F.Cu") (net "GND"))
 (via (at 71.775735 85.624265) (size 0.6) (drill 0.3) (layers "F.Cu" "B.Cu") (capping no) (covering (front no) (back no))
  (plugging (front no) (back no)) (filling no) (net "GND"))
 (via (at 72.924265 85.075735) (size 0.6) (drill 0.3) (layers "F.Cu" "B.Cu") (capping no) (covering (front no) (back no))
  (plugging (front no) (back no)) (filling no) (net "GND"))
 (segment (start 72.324265 85.075735) (end 71.775735 85.624265) (width 0.2) (layer "B.Cu") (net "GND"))
 (segment (start 72.924265 85.075735) (end 72.324265 85.075735) (width 0.2) (layer "B.Cu") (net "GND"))
 (segment (start 72.73 92.7075) (end 72.73 89.53) (width 0.2) (layer "F.Cu") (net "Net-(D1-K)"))
 (segment (start 68.6 89.1875) (end 69.601 88.1865) (width 0.2) (layer "F.Cu") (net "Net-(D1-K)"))
 (segment (start 72.2 89.2) (end 72.1875 89.1875) (width 0.2) (layer "F.Cu") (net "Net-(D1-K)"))
 (segment (start 69.601 88.1865) (end 69.601 85.518499) (width 0.2) (layer "F.Cu") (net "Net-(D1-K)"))
 (segment (start 68.695 84.612499) (end 68.695 83.6375) (width 0.2) (layer "F.Cu") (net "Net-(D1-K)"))
 (segment (start 72.73 89.53) (end 72.4 89.2) (width 0.2) (layer "F.Cu") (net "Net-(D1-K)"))
 (segment (start 72.4 89.2) (end 72.2 89.2) (width 0.2) (layer "F.Cu") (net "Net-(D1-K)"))
 (segment (start 69.601 85.518499) (end 68.695 84.612499) (width 0.2) (layer "F.Cu") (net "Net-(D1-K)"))
 (segment (start 72.1875 89.1875) (end 68.6 89.1875) (width 0.2) (layer "F.Cu") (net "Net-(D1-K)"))
 (segment (start 66.798 85.3355) (end 66.798 74.82834) (width 0.2) (layer "F.Cu") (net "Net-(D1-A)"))
 (segment (start 68.6 87.1375) (end 66.798 85.3355) (width 0.2) (layer "F.Cu") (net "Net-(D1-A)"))
 (segment (start 69.42634 72.2) (end 76.8 72.2) (width 0.2) (layer "F.Cu") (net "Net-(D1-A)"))
 (segment (start 66.798 74.82834) (end 69.42634 72.2) (width 0.2) (layer "F.Cu") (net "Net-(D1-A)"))
 (segment (start 78.1375 73.6) (end 78.3 73.7625) (width 0.2) (layer "F.Cu") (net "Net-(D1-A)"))
 (segment (start 76.8 73.6) (end 78.1375 73.6) (width 0.2) (layer "F.Cu") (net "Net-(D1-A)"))
 (via (at 76.8 73.6) (size 0.6) (drill 0.3) (layers "F.Cu" "B.Cu") (capping no) (covering (front no) (back no))
  (plugging (front no) (back no)) (filling no) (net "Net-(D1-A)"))
 (via (at 76.8 72.2) (size 0.6) (drill 0.3) (layers "F.Cu" "B.Cu") (capping no) (covering (front no) (back no))
  (plugging (front no) (back no)) (filling no) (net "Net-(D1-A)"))
 (segment (start 76.8 72.2) (end 76.8 73.6) (width 0.2) (layer "B.Cu") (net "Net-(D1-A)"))
 (segment (start 80.802 85.5355) (end 79.2 87.1375) (width 0.2) (layer "F.Cu") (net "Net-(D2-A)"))
 (segment (start 78.98516 72.8615) (end 80.802 74.67834) (width 0.2) (layer "F.Cu") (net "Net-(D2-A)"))
 (segment (start 80.802 74.67834) (end 80.802 85.5355) (width 0.2) (layer "F.Cu") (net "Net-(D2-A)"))
 (segment (start 76.251 72.8615) (end 78.98516 72.8615) (width 0.2) (layer "F.Cu") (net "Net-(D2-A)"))
 (segment (start 75.35 73.7625) (end 76.251 72.8615) (width 0.2) (layer "F.Cu") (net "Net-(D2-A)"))
 (segment (start 77.6 83.5125) (end 77.6 83.8) (width 0.2) (layer "F.Cu") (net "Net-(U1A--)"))
 (segment (start 69.965 85.165) (end 69.965 83.6375) (width 0.2) (layer "F.Cu") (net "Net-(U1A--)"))
 (segment (start 70.6 85.8) (end 69.965 85.165) (width 0.2) (layer "F.Cu") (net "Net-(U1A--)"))
 (segment (start 77.6 83.8) (end 76 85.4) (width 0.2) (layer "F.Cu") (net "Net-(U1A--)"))
 (via (at 76 85.4) (size 0.6) (drill 0.3) (layers "F.Cu" "B.Cu") (capping no) (covering (front no) (back no))
  (plugging (front no) (back no)) (filling no) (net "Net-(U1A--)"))
 (via (at 70.6 85.8) (size 0.6) (drill 0.3) (layers "F.Cu" "B.Cu") (capping no) (covering (front no) (back no))
  (plugging (front no) (back no)) (filling no) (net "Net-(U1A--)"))
 (segment (start 76 85.4) (end 75.174735 86.225265) (width 0.2) (layer "B.Cu") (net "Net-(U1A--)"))
 (segment (start 71.025265 86.225265) (end 70.6 85.8) (width 0.2) (layer "B.Cu") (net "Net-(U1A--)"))
 (segment (start 75.174735 86.225265) (end 71.025265 86.225265) (width 0.2) (layer "B.Cu") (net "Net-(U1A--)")))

